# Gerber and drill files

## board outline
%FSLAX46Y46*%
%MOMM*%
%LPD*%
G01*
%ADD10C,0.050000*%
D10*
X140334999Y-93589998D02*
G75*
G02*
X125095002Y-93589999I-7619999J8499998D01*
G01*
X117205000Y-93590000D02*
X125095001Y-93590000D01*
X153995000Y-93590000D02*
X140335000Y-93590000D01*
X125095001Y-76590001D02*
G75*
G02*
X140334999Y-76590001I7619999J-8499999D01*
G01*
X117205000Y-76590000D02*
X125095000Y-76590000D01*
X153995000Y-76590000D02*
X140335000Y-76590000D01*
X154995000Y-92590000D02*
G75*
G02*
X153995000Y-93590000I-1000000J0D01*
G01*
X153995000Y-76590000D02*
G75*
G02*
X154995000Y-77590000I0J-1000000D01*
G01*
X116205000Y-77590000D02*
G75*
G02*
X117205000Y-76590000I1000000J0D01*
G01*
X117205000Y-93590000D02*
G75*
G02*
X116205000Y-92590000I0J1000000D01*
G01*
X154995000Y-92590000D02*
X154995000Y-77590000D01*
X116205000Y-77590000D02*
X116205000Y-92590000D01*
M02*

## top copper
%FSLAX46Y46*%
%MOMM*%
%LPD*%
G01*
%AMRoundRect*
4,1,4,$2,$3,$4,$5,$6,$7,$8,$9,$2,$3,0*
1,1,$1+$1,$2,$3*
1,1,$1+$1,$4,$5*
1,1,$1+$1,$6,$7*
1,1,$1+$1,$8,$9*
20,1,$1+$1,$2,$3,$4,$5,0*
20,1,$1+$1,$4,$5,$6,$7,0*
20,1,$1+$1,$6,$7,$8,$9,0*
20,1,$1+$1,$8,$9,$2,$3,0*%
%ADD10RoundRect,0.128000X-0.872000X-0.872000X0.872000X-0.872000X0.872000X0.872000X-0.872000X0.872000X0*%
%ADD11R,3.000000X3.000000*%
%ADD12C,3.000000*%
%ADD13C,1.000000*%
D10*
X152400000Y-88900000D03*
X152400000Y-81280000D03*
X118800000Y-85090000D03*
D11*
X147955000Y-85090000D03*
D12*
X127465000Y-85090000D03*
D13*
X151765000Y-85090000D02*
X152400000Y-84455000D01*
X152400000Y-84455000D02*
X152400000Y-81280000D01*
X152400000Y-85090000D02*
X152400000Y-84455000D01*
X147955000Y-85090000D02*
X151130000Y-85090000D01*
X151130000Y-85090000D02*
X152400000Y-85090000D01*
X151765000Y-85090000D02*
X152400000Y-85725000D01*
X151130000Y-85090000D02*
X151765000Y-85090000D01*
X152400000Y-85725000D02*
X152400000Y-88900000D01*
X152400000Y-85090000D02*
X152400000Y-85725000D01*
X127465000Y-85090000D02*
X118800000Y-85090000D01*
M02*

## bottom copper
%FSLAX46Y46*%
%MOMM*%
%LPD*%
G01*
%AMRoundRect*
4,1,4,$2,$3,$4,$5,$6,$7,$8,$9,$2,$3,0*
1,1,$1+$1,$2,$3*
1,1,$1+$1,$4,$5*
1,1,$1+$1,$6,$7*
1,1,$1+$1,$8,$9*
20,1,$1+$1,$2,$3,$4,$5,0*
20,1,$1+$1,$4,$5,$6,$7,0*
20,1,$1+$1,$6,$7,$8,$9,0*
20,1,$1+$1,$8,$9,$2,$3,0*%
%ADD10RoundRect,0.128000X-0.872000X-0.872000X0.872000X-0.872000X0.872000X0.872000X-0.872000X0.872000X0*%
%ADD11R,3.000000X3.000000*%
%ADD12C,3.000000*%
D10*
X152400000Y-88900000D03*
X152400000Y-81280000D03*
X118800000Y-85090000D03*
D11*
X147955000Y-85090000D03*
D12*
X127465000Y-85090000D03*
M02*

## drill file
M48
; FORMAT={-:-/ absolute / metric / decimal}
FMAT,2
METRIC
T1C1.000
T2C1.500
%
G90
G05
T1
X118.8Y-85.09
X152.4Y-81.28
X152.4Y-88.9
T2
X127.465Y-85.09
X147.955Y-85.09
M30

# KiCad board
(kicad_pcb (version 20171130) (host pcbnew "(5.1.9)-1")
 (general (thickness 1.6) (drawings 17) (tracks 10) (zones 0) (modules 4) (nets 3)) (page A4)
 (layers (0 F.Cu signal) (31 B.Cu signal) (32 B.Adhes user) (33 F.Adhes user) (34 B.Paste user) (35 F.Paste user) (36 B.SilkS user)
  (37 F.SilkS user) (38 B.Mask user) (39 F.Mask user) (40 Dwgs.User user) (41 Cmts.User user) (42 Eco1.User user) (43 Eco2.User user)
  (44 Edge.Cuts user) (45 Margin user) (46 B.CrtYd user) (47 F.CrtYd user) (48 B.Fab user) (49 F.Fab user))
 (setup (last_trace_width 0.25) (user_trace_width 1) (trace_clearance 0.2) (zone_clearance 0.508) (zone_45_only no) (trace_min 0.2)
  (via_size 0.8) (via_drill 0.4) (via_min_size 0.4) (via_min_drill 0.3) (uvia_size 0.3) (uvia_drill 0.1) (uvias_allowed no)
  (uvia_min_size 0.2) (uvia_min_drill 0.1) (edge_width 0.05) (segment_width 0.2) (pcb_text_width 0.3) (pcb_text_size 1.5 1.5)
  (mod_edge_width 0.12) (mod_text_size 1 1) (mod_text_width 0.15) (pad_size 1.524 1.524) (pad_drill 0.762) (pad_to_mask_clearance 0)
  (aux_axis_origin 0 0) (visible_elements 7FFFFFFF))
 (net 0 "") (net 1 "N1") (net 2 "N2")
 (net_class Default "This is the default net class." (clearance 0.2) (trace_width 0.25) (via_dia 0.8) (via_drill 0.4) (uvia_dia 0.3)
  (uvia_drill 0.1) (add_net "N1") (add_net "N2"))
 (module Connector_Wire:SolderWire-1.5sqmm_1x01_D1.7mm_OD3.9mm (layer F.Cu) (at 152.4 88.9)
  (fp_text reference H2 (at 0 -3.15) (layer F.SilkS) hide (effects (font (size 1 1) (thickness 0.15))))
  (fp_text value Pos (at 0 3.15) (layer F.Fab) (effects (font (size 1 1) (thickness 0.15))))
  (pad 1 thru_hole roundrect (at 0 0) (size 2 2) (drill 1) (layers *.Cu *.Mask) (roundrect_rratio 0.064) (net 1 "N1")))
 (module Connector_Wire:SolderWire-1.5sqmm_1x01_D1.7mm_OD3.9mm (layer F.Cu) (at 152.4 81.28)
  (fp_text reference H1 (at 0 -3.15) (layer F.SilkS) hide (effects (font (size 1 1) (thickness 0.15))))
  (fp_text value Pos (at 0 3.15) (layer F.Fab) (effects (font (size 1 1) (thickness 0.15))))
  (pad 1 thru_hole roundrect (at 0 0) (size 2 2) (drill 1) (layers *.Cu *.Mask) (roundrect_rratio 0.064) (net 1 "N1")))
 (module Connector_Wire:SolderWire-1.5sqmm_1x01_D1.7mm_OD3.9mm (layer F.Cu) (at 118.8 85.09)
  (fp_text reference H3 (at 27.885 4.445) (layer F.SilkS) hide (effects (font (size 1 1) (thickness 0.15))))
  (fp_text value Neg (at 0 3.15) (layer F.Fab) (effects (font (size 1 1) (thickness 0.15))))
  (pad 1 thru_hole roundrect (at 0 0) (size 2 2) (drill 1) (layers *.Cu *.Mask) (roundrect_rratio 0.064) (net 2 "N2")))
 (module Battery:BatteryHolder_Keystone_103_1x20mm (layer F.Cu) (at 147.955 85.09 180)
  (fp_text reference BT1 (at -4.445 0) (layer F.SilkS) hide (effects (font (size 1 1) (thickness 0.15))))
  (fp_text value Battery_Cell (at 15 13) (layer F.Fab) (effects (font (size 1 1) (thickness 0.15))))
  (pad 1 thru_hole rect (at 0 0 180) (size 3 3) (drill 1.5) (layers *.Cu *.Mask) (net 1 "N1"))
  (pad 2 thru_hole circle (at 20.49 0 180) (size 3 3) (drill 1.5) (layers *.Cu *.Mask) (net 2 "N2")))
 (gr_arc (start 132.715 85.09) (end 125.095002 93.589999) (angle -83.75058075) (layer Edge.Cuts) (width 0.05))
 (gr_line (start 117.205 93.59) (end 125.095001 93.59) (layer Edge.Cuts) (width 0.05))
 (gr_line (start 153.995 93.59) (end 140.335 93.59) (layer Edge.Cuts) (width 0.05))
 (gr_arc (start 132.715 85.09) (end 140.334999 76.590001) (angle -83.75058449) (layer Edge.Cuts) (width 0.05))
 (gr_line (start 117.205 76.59) (end 125.095 76.59) (layer Edge.Cuts) (width 0.05))
 (gr_line (start 153.995 76.59) (end 140.335 76.59) (layer Edge.Cuts) (width 0.05))
 (gr_arc (start 153.995 92.59) (end 153.995 93.59) (angle -90) (layer Edge.Cuts) (width 0.05))
 (gr_arc (start 153.995 77.59) (end 154.995 77.59) (angle -90) (layer Edge.Cuts) (width 0.05))
 (gr_arc (start 117.205 77.59) (end 117.205 76.59) (angle -90) (layer Edge.Cuts) (width 0.05))
 (gr_arc (start 117.205 92.59) (end 116.205 92.59) (angle -90) (layer Edge.Cuts) (width 0.05))
 (gr_line (start 154.995 92.59) (end 154.995 77.59) (layer Edge.Cuts) (width 0.05))
 (gr_line (start 116.205 77.59) (end 116.205 92.59) (layer Edge.Cuts) (width 0.05))
 (segment (start 151.765 85.09) (end 152.4 84.455) (width 1) (layer F.Cu) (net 1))
 (segment (start 152.4 84.455) (end 152.4 81.28) (width 1) (layer F.Cu) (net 1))
 (segment (start 152.4 85.09) (end 152.4 84.455) (width 1) (layer F.Cu) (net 1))
 (segment (start 147.955 85.09) (end 151.13 85.09) (width 1) (layer F.Cu) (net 1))
 (segment (start 151.13 85.09) (end 152.4 85.09) (width 1) (layer F.Cu) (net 1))
 (segment (start 151.765 85.09) (end 152.4 85.725) (width 1) (layer F.Cu) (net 1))
 (segment (start 151.13 85.09) (end 151.765 85.09) (width 1) (layer F.Cu) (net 1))
 (segment (start 152.4 85.725) (end 152.4 88.9) (width 1) (layer F.Cu) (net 1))
 (segment (start 152.4 85.09) (end 152.4 85.725) (width 1) (layer F.Cu) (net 1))
 (segment (start 127.465 85.09) (end 118.8 85.09) (width 1) (layer F.Cu) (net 2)))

